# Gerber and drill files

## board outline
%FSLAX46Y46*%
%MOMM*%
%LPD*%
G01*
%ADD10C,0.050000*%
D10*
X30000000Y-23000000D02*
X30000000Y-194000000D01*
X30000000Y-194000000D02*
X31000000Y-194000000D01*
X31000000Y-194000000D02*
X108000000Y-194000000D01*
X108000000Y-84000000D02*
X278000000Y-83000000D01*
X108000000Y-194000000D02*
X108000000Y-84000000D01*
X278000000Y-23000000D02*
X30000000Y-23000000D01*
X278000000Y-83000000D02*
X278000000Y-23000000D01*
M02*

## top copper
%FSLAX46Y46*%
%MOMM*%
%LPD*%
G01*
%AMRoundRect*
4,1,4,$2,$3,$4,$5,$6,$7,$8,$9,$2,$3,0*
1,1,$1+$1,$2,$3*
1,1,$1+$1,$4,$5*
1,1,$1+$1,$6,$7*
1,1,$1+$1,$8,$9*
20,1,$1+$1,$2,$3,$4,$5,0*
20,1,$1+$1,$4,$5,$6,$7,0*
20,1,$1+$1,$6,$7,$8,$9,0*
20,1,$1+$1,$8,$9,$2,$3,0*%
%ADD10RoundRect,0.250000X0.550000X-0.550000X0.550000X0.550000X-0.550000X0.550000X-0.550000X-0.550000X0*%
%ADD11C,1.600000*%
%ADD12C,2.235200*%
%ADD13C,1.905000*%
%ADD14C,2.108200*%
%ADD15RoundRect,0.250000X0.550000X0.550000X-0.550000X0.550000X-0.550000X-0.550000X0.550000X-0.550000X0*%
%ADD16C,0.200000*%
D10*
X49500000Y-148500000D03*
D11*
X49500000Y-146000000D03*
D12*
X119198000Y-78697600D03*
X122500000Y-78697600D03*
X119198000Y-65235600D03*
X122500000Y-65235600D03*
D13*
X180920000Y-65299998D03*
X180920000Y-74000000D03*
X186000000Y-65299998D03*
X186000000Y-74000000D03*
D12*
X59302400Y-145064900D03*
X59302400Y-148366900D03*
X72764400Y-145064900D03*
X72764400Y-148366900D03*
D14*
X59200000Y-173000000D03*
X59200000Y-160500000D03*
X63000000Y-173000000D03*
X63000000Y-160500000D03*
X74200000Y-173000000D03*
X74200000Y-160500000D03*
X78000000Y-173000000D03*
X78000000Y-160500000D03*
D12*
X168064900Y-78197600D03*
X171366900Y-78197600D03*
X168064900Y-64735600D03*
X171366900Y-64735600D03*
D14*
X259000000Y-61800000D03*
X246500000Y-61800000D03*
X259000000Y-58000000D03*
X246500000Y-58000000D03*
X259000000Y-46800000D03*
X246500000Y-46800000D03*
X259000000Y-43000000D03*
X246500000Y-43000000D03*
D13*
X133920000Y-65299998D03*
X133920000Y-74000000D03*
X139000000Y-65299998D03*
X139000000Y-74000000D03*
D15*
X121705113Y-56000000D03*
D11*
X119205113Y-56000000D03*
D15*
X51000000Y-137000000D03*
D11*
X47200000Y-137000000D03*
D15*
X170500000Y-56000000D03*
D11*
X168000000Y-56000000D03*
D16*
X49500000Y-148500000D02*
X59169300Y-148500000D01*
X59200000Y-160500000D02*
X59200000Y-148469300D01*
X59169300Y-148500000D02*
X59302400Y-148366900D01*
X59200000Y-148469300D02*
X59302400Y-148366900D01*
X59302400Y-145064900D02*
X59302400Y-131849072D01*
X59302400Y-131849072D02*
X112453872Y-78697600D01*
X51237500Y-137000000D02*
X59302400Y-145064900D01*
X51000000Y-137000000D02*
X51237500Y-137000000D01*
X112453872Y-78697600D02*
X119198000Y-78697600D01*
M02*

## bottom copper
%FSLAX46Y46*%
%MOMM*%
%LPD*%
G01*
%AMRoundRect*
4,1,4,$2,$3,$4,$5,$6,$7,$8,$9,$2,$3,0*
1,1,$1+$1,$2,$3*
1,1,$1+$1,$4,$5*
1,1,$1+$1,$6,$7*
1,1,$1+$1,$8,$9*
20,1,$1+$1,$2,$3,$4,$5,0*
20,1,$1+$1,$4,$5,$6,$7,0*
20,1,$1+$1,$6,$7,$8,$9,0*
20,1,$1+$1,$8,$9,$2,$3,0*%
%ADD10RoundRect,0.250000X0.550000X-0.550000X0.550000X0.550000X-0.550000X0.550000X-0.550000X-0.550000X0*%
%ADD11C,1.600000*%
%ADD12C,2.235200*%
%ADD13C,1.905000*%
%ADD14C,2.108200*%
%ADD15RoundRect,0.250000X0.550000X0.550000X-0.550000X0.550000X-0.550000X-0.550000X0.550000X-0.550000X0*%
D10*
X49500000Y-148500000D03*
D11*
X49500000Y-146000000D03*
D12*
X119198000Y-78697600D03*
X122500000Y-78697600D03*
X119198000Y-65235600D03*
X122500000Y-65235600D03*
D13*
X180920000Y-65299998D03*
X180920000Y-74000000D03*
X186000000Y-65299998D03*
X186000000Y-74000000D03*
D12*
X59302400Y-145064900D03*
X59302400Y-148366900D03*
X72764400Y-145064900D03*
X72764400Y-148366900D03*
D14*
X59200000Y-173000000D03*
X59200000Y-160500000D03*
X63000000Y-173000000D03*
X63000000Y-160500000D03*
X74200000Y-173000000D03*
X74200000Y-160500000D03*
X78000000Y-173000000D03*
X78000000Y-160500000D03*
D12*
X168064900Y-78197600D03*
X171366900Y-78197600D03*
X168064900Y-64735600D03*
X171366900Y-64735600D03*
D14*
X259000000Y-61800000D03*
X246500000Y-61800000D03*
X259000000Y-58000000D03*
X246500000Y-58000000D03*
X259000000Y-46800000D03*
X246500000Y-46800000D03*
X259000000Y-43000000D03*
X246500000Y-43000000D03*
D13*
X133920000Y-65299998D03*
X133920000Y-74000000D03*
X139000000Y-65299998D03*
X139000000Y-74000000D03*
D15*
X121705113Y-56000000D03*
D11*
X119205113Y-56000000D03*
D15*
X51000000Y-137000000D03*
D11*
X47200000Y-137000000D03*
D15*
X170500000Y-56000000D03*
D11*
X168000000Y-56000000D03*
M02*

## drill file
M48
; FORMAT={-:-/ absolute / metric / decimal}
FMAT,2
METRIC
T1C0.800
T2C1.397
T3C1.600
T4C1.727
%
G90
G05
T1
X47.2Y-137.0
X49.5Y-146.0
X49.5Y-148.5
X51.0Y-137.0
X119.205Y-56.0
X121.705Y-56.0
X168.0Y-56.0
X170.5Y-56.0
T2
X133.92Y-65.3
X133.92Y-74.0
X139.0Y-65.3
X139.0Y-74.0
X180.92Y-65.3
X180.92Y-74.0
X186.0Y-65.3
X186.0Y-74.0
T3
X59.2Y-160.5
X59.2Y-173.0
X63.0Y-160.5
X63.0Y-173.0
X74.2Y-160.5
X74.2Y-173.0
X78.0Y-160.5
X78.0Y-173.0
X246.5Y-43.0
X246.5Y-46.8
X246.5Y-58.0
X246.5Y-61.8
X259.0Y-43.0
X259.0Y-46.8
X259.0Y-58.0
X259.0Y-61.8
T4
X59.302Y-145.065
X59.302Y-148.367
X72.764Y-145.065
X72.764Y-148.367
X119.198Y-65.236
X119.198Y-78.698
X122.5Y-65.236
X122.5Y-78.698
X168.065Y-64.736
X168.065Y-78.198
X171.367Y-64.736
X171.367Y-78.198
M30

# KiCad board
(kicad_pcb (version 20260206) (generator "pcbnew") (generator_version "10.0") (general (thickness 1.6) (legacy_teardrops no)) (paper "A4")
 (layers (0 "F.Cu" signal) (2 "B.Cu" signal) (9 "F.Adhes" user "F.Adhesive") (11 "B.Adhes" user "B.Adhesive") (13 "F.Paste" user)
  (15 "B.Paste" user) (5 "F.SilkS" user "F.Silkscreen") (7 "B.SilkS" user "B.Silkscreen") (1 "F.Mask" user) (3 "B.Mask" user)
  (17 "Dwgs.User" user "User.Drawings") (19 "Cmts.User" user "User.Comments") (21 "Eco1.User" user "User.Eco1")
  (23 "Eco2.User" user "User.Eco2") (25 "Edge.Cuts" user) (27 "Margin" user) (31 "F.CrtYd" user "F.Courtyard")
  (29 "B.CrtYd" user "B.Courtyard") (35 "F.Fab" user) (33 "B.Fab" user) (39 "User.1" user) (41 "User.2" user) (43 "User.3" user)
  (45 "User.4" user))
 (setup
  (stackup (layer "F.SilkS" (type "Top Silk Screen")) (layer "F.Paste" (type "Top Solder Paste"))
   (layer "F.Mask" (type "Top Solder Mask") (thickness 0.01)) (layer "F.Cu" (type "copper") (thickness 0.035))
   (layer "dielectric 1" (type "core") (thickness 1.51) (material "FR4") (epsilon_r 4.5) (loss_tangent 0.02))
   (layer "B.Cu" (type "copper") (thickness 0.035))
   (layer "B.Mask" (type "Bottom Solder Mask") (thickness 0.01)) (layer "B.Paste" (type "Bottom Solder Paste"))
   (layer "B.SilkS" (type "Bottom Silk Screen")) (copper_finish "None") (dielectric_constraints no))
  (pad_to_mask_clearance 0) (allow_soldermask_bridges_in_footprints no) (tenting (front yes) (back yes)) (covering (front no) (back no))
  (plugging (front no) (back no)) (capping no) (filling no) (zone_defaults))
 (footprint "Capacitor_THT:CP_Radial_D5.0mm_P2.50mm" (layer "F.Cu") (at 49.5 148.5 90)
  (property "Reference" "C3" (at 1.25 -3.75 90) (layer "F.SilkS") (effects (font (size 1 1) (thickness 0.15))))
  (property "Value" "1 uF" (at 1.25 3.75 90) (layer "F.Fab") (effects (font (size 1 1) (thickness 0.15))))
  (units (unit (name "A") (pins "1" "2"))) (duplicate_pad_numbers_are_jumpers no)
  (pad "1" thru_hole roundrect (at 0 0 90) (size 1.6 1.6) (drill 0.8) (layers "*.Cu" "*.Mask") (remove_unused_layers no)
   (roundrect_rratio 0.15625) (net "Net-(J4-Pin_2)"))
  (pad "2" thru_hole circle (at 2.5 0 90) (size 1.6 1.6) (drill 0.8) (layers "*.Cu" "*.Mask") (remove_unused_layers no) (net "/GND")))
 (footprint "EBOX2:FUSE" (layer "F.Cu") (at 119.198 78.6976 90)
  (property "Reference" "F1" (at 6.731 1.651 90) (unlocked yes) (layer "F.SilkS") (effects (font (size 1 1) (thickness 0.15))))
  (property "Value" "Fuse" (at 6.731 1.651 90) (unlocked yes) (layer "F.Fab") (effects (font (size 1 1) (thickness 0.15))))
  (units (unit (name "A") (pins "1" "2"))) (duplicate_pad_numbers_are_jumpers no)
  (pad "1" thru_hole circle (at 0 0 90) (size 2.2352 2.2352) (drill 1.7272) (layers "*.Cu" "*.Mask") (remove_unused_layers no)
   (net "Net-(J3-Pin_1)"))
  (pad "2" thru_hole circle (at 0 3.302 90) (size 2.2352 2.2352) (drill 1.7272) (layers "*.Cu" "*.Mask") (remove_unused_layers no)
   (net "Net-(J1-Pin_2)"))
  (pad "3" thru_hole circle (at 13.462 0 90) (size 2.2352 2.2352) (drill 1.7272) (layers "*.Cu" "*.Mask") (remove_unused_layers no))
  (pad "4" thru_hole circle (at 13.462 3.302 90) (size 2.2352 2.2352) (drill 1.7272) (layers "*.Cu" "*.Mask") (remove_unused_layers no)))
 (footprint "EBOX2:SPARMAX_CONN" (layer "F.Cu") (at 186 74)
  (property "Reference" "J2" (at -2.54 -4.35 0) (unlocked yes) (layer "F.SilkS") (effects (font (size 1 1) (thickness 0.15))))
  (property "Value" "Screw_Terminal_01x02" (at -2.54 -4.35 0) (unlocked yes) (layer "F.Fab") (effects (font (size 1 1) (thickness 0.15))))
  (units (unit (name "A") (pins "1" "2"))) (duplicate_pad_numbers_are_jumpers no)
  (pad "1" thru_hole circle (at -5.08 -8.700002) (size 1.905 1.905) (drill 1.397) (layers "*.Cu" "*.Mask") (remove_unused_layers no)
   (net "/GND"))
  (pad "2" thru_hole circle (at -5.08 0) (size 1.905 1.905) (drill 1.397) (layers "*.Cu" "*.Mask") (remove_unused_layers no)
   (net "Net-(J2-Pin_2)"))
  (pad "3" thru_hole circle (at 0 -8.700002) (size 1.905 1.905) (drill 1.397) (layers "*.Cu" "*.Mask") (remove_unused_layers no))
  (pad "4" thru_hole circle (at 0 0) (size 1.905 1.905) (drill 1.397) (layers "*.Cu" "*.Mask") (remove_unused_layers no)))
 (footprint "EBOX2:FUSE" (layer "F.Cu") (at 59.3024 145.0649)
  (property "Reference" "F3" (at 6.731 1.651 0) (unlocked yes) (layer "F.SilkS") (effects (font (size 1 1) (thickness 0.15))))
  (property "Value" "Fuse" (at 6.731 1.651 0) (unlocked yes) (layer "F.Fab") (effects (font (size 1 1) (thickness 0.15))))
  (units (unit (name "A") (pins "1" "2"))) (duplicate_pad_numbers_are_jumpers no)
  (pad "1" thru_hole circle (at 0 0) (size 2.2352 2.2352) (drill 1.7272) (layers "*.Cu" "*.Mask") (remove_unused_layers no)
   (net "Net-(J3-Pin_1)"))
  (pad "2" thru_hole circle (at 0 3.302) (size 2.2352 2.2352) (drill 1.7272) (layers "*.Cu" "*.Mask") (remove_unused_layers no)
   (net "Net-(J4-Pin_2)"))
  (pad "3" thru_hole circle (at 13.462 0) (size 2.2352 2.2352) (drill 1.7272) (layers "*.Cu" "*.Mask") (remove_unused_layers no))
  (pad "4" thru_hole circle (at 13.462 3.302) (size 2.2352 2.2352) (drill 1.7272) (layers "*.Cu" "*.Mask") (remove_unused_layers no)))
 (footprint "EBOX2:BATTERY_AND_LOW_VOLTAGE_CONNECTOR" (layer "F.Cu") (at 59.2 173)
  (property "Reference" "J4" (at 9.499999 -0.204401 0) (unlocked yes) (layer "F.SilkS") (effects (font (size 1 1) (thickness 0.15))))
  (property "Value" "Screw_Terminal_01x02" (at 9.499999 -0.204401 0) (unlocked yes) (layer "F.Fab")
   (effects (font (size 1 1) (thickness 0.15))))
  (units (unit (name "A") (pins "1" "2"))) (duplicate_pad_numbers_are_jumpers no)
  (pad "1" thru_hole circle (at 0 0) (size 2.1082 2.1082) (drill 1.6002) (layers "*.Cu" "*.Mask") (remove_unused_layers no) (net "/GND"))
  (pad "2" thru_hole circle (at 0 -12.5) (size 2.1082 2.1082) (drill 1.6002) (layers "*.Cu" "*.Mask") (remove_unused_layers no)
   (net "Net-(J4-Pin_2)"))
  (pad "3" thru_hole circle (at 3.8 0) (size 2.1082 2.1082) (drill 1.6002) (layers "*.Cu" "*.Mask") (remove_unused_layers no))
  (pad "4" thru_hole circle (at 3.8 -12.5) (size 2.1082 2.1082) (drill 1.6002) (layers "*.Cu" "*.Mask") (remove_unused_layers no))
  (pad "5" thru_hole circle (at 15 0) (size 2.1082 2.1082) (drill 1.6002) (layers "*.Cu" "*.Mask") (remove_unused_layers no))
  (pad "6" thru_hole circle (at 15 -12.5) (size 2.1082 2.1082) (drill 1.6002) (layers "*.Cu" "*.Mask") (remove_unused_layers no))
  (pad "7" thru_hole circle (at 18.8 0) (size 2.1082 2.1082) (drill 1.6002) (layers "*.Cu" "*.Mask") (remove_unused_layers no))
  (pad "8" thru_hole circle (at 18.8 -12.5) (size 2.1082 2.1082) (drill 1.6002) (layers "*.Cu" "*.Mask") (remove_unused_layers no)))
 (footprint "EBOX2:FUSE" (layer "F.Cu") (at 168.0649 78.1976 90)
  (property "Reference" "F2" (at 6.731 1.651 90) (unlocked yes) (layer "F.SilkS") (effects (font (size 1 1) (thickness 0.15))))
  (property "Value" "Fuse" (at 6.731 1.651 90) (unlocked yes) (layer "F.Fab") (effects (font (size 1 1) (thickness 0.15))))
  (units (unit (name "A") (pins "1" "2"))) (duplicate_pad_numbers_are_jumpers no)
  (pad "1" thru_hole circle (at 0 0 90) (size 2.2352 2.2352) (drill 1.7272) (layers "*.Cu" "*.Mask") (remove_unused_layers no)
   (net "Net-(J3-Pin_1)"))
  (pad "2" thru_hole circle (at 0 3.302 90) (size 2.2352 2.2352) (drill 1.7272) (layers "*.Cu" "*.Mask") (remove_unused_layers no)
   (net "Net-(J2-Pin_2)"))
  (pad "3" thru_hole circle (at 13.462 0 90) (size 2.2352 2.2352) (drill 1.7272) (layers "*.Cu" "*.Mask") (remove_unused_layers no))
  (pad "4" thru_hole circle (at 13.462 3.302 90) (size 2.2352 2.2352) (drill 1.7272) (layers "*.Cu" "*.Mask") (remove_unused_layers no)))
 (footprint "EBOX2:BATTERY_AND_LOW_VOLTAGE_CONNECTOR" (layer "F.Cu") (at 259 61.8 90)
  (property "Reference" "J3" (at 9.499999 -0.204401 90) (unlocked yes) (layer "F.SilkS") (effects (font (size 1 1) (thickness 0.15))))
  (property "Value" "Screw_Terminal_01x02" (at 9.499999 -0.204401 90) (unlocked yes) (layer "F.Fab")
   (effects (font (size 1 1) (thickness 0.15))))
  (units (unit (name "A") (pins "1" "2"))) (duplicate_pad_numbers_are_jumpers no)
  (pad "1" thru_hole circle (at 0 0 90) (size 2.1082 2.1082) (drill 1.6002) (layers "*.Cu" "*.Mask") (remove_unused_layers no)
   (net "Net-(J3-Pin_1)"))
  (pad "2" thru_hole circle (at 0 -12.5 90) (size 2.1082 2.1082) (drill 1.6002) (layers "*.Cu" "*.Mask") (remove_unused_layers no)
   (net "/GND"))
  (pad "3" thru_hole circle (at 3.8 0 90) (size 2.1082 2.1082) (drill 1.6002) (layers "*.Cu" "*.Mask") (remove_unused_layers no))
  (pad "4" thru_hole circle (at 3.8 -12.5 90) (size 2.1082 2.1082) (drill 1.6002) (layers "*.Cu" "*.Mask") (remove_unused_layers no))
  (pad "5" thru_hole circle (at 15 0 90) (size 2.1082 2.1082) (drill 1.6002) (layers "*.Cu" "*.Mask") (remove_unused_layers no))
  (pad "6" thru_hole circle (at 15 -12.5 90) (size 2.1082 2.1082) (drill 1.6002) (layers "*.Cu" "*.Mask") (remove_unused_layers no))
  (pad "7" thru_hole circle (at 18.8 0 90) (size 2.1082 2.1082) (drill 1.6002) (layers "*.Cu" "*.Mask") (remove_unused_layers no))
  (pad "8" thru_hole circle (at 18.8 -12.5 90) (size 2.1082 2.1082) (drill 1.6002) (layers "*.Cu" "*.Mask") (remove_unused_layers no)))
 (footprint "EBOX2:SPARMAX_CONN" (layer "F.Cu") (at 139 74)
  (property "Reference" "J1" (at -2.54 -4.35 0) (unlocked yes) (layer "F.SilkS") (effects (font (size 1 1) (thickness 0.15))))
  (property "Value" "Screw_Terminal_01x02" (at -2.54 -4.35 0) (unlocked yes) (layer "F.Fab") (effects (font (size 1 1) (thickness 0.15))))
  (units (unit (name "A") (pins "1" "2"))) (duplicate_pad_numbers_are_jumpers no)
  (pad "1" thru_hole circle (at -5.08 -8.700002) (size 1.905 1.905) (drill 1.397) (layers "*.Cu" "*.Mask") (remove_unused_layers no)
   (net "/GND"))
  (pad "2" thru_hole circle (at -5.08 0) (size 1.905 1.905) (drill 1.397) (layers "*.Cu" "*.Mask") (remove_unused_layers no)
   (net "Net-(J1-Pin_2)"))
  (pad "3" thru_hole circle (at 0 -8.700002) (size 1.905 1.905) (drill 1.397) (layers "*.Cu" "*.Mask") (remove_unused_layers no))
  (pad "4" thru_hole circle (at 0 0) (size 1.905 1.905) (drill 1.397) (layers "*.Cu" "*.Mask") (remove_unused_layers no)))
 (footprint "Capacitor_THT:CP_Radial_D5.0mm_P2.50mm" (layer "F.Cu") (at 121.705113 56 180)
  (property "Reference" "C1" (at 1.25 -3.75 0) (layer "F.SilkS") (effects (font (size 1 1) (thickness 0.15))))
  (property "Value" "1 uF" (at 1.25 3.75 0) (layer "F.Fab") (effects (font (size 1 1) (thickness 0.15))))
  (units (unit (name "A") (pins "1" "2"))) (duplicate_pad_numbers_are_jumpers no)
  (pad "1" thru_hole roundrect (at 0 0 180) (size 1.6 1.6) (drill 0.8) (layers "*.Cu" "*.Mask") (remove_unused_layers no)
   (roundrect_rratio 0.15625) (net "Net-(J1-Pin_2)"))
  (pad "2" thru_hole circle (at 2.5 0 180) (size 1.6 1.6) (drill 0.8) (layers "*.Cu" "*.Mask") (remove_unused_layers no) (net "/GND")))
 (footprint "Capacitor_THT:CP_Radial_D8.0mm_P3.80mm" (layer "F.Cu") (at 51 137 180)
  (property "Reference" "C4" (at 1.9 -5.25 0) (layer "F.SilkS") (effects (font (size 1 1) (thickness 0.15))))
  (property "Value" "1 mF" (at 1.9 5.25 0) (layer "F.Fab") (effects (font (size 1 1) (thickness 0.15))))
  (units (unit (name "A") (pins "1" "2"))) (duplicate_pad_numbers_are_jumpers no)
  (pad "1" thru_hole roundrect (at 0 0 180) (size 1.6 1.6) (drill 0.8) (layers "*.Cu" "*.Mask") (remove_unused_layers no)
   (roundrect_rratio 0.15625) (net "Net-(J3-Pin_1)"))
  (pad "2" thru_hole circle (at 3.8 0 180) (size 1.6 1.6) (drill 0.8) (layers "*.Cu" "*.Mask") (remove_unused_layers no) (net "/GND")))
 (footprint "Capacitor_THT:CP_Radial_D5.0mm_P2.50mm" (layer "F.Cu") (at 170.5 56 180)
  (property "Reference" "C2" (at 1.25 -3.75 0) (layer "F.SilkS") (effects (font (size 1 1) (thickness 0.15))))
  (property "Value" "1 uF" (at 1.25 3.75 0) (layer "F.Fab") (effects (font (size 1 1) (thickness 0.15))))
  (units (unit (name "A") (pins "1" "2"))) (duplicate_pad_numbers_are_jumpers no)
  (pad "1" thru_hole roundrect (at 0 0 180) (size 1.6 1.6) (drill 0.8) (layers "*.Cu" "*.Mask") (remove_unused_layers no)
   (roundrect_rratio 0.15625) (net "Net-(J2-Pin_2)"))
  (pad "2" thru_hole circle (at 2.5 0 180) (size 1.6 1.6) (drill 0.8) (layers "*.Cu" "*.Mask") (remove_unused_layers no) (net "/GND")))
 (gr_line (start 30 23) (end 30 194) (stroke (width 0.05) (type default)) (layer "Edge.Cuts"))
 (gr_line (start 30 194) (end 31 194) (stroke (width 0.05) (type default)) (layer "Edge.Cuts"))
 (gr_line (start 31 194) (end 108 194) (stroke (width 0.05) (type default)) (layer "Edge.Cuts"))
 (gr_line (start 108 84) (end 278 83) (stroke (width 0.05) (type default)) (layer "Edge.Cuts"))
 (gr_line (start 108 194) (end 108 84) (stroke (width 0.05) (type default)) (layer "Edge.Cuts"))
 (gr_line (start 278 23) (end 30 23) (stroke (width 0.05) (type default)) (layer "Edge.Cuts"))
 (gr_line (start 278 83) (end 278 23) (stroke (width 0.05) (type default)) (layer "Edge.Cuts"))
 (segment (start 49.5 148.5) (end 59.1693 148.5) (width 0.2) (layer "F.Cu") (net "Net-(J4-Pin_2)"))
 (segment (start 59.2 160.5) (end 59.2 148.4693) (width 0.2) (layer "F.Cu") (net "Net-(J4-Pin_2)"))
 (segment (start 59.1693 148.5) (end 59.3024 148.3669) (width 0.2) (layer "F.Cu") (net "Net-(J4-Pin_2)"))
 (segment (start 59.2 148.4693) (end 59.3024 148.3669) (width 0.2) (layer "F.Cu") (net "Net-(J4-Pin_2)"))
 (segment (start 59.3024 145.0649) (end 59.3024 131.849072) (width 0.2) (layer "F.Cu") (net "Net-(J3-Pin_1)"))
 (segment (start 59.3024 131.849072) (end 112.453872 78.6976) (width 0.2) (layer "F.Cu") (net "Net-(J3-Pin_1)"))
 (segment (start 51.2375 137) (end 59.3024 145.0649) (width 0.2) (layer "F.Cu") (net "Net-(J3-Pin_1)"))
 (segment (start 51 137) (end 51.2375 137) (width 0.2) (layer "F.Cu") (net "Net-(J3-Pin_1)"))
 (segment (start 112.453872 78.6976) (end 119.198 78.6976) (width 0.2) (layer "F.Cu") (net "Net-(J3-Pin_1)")))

